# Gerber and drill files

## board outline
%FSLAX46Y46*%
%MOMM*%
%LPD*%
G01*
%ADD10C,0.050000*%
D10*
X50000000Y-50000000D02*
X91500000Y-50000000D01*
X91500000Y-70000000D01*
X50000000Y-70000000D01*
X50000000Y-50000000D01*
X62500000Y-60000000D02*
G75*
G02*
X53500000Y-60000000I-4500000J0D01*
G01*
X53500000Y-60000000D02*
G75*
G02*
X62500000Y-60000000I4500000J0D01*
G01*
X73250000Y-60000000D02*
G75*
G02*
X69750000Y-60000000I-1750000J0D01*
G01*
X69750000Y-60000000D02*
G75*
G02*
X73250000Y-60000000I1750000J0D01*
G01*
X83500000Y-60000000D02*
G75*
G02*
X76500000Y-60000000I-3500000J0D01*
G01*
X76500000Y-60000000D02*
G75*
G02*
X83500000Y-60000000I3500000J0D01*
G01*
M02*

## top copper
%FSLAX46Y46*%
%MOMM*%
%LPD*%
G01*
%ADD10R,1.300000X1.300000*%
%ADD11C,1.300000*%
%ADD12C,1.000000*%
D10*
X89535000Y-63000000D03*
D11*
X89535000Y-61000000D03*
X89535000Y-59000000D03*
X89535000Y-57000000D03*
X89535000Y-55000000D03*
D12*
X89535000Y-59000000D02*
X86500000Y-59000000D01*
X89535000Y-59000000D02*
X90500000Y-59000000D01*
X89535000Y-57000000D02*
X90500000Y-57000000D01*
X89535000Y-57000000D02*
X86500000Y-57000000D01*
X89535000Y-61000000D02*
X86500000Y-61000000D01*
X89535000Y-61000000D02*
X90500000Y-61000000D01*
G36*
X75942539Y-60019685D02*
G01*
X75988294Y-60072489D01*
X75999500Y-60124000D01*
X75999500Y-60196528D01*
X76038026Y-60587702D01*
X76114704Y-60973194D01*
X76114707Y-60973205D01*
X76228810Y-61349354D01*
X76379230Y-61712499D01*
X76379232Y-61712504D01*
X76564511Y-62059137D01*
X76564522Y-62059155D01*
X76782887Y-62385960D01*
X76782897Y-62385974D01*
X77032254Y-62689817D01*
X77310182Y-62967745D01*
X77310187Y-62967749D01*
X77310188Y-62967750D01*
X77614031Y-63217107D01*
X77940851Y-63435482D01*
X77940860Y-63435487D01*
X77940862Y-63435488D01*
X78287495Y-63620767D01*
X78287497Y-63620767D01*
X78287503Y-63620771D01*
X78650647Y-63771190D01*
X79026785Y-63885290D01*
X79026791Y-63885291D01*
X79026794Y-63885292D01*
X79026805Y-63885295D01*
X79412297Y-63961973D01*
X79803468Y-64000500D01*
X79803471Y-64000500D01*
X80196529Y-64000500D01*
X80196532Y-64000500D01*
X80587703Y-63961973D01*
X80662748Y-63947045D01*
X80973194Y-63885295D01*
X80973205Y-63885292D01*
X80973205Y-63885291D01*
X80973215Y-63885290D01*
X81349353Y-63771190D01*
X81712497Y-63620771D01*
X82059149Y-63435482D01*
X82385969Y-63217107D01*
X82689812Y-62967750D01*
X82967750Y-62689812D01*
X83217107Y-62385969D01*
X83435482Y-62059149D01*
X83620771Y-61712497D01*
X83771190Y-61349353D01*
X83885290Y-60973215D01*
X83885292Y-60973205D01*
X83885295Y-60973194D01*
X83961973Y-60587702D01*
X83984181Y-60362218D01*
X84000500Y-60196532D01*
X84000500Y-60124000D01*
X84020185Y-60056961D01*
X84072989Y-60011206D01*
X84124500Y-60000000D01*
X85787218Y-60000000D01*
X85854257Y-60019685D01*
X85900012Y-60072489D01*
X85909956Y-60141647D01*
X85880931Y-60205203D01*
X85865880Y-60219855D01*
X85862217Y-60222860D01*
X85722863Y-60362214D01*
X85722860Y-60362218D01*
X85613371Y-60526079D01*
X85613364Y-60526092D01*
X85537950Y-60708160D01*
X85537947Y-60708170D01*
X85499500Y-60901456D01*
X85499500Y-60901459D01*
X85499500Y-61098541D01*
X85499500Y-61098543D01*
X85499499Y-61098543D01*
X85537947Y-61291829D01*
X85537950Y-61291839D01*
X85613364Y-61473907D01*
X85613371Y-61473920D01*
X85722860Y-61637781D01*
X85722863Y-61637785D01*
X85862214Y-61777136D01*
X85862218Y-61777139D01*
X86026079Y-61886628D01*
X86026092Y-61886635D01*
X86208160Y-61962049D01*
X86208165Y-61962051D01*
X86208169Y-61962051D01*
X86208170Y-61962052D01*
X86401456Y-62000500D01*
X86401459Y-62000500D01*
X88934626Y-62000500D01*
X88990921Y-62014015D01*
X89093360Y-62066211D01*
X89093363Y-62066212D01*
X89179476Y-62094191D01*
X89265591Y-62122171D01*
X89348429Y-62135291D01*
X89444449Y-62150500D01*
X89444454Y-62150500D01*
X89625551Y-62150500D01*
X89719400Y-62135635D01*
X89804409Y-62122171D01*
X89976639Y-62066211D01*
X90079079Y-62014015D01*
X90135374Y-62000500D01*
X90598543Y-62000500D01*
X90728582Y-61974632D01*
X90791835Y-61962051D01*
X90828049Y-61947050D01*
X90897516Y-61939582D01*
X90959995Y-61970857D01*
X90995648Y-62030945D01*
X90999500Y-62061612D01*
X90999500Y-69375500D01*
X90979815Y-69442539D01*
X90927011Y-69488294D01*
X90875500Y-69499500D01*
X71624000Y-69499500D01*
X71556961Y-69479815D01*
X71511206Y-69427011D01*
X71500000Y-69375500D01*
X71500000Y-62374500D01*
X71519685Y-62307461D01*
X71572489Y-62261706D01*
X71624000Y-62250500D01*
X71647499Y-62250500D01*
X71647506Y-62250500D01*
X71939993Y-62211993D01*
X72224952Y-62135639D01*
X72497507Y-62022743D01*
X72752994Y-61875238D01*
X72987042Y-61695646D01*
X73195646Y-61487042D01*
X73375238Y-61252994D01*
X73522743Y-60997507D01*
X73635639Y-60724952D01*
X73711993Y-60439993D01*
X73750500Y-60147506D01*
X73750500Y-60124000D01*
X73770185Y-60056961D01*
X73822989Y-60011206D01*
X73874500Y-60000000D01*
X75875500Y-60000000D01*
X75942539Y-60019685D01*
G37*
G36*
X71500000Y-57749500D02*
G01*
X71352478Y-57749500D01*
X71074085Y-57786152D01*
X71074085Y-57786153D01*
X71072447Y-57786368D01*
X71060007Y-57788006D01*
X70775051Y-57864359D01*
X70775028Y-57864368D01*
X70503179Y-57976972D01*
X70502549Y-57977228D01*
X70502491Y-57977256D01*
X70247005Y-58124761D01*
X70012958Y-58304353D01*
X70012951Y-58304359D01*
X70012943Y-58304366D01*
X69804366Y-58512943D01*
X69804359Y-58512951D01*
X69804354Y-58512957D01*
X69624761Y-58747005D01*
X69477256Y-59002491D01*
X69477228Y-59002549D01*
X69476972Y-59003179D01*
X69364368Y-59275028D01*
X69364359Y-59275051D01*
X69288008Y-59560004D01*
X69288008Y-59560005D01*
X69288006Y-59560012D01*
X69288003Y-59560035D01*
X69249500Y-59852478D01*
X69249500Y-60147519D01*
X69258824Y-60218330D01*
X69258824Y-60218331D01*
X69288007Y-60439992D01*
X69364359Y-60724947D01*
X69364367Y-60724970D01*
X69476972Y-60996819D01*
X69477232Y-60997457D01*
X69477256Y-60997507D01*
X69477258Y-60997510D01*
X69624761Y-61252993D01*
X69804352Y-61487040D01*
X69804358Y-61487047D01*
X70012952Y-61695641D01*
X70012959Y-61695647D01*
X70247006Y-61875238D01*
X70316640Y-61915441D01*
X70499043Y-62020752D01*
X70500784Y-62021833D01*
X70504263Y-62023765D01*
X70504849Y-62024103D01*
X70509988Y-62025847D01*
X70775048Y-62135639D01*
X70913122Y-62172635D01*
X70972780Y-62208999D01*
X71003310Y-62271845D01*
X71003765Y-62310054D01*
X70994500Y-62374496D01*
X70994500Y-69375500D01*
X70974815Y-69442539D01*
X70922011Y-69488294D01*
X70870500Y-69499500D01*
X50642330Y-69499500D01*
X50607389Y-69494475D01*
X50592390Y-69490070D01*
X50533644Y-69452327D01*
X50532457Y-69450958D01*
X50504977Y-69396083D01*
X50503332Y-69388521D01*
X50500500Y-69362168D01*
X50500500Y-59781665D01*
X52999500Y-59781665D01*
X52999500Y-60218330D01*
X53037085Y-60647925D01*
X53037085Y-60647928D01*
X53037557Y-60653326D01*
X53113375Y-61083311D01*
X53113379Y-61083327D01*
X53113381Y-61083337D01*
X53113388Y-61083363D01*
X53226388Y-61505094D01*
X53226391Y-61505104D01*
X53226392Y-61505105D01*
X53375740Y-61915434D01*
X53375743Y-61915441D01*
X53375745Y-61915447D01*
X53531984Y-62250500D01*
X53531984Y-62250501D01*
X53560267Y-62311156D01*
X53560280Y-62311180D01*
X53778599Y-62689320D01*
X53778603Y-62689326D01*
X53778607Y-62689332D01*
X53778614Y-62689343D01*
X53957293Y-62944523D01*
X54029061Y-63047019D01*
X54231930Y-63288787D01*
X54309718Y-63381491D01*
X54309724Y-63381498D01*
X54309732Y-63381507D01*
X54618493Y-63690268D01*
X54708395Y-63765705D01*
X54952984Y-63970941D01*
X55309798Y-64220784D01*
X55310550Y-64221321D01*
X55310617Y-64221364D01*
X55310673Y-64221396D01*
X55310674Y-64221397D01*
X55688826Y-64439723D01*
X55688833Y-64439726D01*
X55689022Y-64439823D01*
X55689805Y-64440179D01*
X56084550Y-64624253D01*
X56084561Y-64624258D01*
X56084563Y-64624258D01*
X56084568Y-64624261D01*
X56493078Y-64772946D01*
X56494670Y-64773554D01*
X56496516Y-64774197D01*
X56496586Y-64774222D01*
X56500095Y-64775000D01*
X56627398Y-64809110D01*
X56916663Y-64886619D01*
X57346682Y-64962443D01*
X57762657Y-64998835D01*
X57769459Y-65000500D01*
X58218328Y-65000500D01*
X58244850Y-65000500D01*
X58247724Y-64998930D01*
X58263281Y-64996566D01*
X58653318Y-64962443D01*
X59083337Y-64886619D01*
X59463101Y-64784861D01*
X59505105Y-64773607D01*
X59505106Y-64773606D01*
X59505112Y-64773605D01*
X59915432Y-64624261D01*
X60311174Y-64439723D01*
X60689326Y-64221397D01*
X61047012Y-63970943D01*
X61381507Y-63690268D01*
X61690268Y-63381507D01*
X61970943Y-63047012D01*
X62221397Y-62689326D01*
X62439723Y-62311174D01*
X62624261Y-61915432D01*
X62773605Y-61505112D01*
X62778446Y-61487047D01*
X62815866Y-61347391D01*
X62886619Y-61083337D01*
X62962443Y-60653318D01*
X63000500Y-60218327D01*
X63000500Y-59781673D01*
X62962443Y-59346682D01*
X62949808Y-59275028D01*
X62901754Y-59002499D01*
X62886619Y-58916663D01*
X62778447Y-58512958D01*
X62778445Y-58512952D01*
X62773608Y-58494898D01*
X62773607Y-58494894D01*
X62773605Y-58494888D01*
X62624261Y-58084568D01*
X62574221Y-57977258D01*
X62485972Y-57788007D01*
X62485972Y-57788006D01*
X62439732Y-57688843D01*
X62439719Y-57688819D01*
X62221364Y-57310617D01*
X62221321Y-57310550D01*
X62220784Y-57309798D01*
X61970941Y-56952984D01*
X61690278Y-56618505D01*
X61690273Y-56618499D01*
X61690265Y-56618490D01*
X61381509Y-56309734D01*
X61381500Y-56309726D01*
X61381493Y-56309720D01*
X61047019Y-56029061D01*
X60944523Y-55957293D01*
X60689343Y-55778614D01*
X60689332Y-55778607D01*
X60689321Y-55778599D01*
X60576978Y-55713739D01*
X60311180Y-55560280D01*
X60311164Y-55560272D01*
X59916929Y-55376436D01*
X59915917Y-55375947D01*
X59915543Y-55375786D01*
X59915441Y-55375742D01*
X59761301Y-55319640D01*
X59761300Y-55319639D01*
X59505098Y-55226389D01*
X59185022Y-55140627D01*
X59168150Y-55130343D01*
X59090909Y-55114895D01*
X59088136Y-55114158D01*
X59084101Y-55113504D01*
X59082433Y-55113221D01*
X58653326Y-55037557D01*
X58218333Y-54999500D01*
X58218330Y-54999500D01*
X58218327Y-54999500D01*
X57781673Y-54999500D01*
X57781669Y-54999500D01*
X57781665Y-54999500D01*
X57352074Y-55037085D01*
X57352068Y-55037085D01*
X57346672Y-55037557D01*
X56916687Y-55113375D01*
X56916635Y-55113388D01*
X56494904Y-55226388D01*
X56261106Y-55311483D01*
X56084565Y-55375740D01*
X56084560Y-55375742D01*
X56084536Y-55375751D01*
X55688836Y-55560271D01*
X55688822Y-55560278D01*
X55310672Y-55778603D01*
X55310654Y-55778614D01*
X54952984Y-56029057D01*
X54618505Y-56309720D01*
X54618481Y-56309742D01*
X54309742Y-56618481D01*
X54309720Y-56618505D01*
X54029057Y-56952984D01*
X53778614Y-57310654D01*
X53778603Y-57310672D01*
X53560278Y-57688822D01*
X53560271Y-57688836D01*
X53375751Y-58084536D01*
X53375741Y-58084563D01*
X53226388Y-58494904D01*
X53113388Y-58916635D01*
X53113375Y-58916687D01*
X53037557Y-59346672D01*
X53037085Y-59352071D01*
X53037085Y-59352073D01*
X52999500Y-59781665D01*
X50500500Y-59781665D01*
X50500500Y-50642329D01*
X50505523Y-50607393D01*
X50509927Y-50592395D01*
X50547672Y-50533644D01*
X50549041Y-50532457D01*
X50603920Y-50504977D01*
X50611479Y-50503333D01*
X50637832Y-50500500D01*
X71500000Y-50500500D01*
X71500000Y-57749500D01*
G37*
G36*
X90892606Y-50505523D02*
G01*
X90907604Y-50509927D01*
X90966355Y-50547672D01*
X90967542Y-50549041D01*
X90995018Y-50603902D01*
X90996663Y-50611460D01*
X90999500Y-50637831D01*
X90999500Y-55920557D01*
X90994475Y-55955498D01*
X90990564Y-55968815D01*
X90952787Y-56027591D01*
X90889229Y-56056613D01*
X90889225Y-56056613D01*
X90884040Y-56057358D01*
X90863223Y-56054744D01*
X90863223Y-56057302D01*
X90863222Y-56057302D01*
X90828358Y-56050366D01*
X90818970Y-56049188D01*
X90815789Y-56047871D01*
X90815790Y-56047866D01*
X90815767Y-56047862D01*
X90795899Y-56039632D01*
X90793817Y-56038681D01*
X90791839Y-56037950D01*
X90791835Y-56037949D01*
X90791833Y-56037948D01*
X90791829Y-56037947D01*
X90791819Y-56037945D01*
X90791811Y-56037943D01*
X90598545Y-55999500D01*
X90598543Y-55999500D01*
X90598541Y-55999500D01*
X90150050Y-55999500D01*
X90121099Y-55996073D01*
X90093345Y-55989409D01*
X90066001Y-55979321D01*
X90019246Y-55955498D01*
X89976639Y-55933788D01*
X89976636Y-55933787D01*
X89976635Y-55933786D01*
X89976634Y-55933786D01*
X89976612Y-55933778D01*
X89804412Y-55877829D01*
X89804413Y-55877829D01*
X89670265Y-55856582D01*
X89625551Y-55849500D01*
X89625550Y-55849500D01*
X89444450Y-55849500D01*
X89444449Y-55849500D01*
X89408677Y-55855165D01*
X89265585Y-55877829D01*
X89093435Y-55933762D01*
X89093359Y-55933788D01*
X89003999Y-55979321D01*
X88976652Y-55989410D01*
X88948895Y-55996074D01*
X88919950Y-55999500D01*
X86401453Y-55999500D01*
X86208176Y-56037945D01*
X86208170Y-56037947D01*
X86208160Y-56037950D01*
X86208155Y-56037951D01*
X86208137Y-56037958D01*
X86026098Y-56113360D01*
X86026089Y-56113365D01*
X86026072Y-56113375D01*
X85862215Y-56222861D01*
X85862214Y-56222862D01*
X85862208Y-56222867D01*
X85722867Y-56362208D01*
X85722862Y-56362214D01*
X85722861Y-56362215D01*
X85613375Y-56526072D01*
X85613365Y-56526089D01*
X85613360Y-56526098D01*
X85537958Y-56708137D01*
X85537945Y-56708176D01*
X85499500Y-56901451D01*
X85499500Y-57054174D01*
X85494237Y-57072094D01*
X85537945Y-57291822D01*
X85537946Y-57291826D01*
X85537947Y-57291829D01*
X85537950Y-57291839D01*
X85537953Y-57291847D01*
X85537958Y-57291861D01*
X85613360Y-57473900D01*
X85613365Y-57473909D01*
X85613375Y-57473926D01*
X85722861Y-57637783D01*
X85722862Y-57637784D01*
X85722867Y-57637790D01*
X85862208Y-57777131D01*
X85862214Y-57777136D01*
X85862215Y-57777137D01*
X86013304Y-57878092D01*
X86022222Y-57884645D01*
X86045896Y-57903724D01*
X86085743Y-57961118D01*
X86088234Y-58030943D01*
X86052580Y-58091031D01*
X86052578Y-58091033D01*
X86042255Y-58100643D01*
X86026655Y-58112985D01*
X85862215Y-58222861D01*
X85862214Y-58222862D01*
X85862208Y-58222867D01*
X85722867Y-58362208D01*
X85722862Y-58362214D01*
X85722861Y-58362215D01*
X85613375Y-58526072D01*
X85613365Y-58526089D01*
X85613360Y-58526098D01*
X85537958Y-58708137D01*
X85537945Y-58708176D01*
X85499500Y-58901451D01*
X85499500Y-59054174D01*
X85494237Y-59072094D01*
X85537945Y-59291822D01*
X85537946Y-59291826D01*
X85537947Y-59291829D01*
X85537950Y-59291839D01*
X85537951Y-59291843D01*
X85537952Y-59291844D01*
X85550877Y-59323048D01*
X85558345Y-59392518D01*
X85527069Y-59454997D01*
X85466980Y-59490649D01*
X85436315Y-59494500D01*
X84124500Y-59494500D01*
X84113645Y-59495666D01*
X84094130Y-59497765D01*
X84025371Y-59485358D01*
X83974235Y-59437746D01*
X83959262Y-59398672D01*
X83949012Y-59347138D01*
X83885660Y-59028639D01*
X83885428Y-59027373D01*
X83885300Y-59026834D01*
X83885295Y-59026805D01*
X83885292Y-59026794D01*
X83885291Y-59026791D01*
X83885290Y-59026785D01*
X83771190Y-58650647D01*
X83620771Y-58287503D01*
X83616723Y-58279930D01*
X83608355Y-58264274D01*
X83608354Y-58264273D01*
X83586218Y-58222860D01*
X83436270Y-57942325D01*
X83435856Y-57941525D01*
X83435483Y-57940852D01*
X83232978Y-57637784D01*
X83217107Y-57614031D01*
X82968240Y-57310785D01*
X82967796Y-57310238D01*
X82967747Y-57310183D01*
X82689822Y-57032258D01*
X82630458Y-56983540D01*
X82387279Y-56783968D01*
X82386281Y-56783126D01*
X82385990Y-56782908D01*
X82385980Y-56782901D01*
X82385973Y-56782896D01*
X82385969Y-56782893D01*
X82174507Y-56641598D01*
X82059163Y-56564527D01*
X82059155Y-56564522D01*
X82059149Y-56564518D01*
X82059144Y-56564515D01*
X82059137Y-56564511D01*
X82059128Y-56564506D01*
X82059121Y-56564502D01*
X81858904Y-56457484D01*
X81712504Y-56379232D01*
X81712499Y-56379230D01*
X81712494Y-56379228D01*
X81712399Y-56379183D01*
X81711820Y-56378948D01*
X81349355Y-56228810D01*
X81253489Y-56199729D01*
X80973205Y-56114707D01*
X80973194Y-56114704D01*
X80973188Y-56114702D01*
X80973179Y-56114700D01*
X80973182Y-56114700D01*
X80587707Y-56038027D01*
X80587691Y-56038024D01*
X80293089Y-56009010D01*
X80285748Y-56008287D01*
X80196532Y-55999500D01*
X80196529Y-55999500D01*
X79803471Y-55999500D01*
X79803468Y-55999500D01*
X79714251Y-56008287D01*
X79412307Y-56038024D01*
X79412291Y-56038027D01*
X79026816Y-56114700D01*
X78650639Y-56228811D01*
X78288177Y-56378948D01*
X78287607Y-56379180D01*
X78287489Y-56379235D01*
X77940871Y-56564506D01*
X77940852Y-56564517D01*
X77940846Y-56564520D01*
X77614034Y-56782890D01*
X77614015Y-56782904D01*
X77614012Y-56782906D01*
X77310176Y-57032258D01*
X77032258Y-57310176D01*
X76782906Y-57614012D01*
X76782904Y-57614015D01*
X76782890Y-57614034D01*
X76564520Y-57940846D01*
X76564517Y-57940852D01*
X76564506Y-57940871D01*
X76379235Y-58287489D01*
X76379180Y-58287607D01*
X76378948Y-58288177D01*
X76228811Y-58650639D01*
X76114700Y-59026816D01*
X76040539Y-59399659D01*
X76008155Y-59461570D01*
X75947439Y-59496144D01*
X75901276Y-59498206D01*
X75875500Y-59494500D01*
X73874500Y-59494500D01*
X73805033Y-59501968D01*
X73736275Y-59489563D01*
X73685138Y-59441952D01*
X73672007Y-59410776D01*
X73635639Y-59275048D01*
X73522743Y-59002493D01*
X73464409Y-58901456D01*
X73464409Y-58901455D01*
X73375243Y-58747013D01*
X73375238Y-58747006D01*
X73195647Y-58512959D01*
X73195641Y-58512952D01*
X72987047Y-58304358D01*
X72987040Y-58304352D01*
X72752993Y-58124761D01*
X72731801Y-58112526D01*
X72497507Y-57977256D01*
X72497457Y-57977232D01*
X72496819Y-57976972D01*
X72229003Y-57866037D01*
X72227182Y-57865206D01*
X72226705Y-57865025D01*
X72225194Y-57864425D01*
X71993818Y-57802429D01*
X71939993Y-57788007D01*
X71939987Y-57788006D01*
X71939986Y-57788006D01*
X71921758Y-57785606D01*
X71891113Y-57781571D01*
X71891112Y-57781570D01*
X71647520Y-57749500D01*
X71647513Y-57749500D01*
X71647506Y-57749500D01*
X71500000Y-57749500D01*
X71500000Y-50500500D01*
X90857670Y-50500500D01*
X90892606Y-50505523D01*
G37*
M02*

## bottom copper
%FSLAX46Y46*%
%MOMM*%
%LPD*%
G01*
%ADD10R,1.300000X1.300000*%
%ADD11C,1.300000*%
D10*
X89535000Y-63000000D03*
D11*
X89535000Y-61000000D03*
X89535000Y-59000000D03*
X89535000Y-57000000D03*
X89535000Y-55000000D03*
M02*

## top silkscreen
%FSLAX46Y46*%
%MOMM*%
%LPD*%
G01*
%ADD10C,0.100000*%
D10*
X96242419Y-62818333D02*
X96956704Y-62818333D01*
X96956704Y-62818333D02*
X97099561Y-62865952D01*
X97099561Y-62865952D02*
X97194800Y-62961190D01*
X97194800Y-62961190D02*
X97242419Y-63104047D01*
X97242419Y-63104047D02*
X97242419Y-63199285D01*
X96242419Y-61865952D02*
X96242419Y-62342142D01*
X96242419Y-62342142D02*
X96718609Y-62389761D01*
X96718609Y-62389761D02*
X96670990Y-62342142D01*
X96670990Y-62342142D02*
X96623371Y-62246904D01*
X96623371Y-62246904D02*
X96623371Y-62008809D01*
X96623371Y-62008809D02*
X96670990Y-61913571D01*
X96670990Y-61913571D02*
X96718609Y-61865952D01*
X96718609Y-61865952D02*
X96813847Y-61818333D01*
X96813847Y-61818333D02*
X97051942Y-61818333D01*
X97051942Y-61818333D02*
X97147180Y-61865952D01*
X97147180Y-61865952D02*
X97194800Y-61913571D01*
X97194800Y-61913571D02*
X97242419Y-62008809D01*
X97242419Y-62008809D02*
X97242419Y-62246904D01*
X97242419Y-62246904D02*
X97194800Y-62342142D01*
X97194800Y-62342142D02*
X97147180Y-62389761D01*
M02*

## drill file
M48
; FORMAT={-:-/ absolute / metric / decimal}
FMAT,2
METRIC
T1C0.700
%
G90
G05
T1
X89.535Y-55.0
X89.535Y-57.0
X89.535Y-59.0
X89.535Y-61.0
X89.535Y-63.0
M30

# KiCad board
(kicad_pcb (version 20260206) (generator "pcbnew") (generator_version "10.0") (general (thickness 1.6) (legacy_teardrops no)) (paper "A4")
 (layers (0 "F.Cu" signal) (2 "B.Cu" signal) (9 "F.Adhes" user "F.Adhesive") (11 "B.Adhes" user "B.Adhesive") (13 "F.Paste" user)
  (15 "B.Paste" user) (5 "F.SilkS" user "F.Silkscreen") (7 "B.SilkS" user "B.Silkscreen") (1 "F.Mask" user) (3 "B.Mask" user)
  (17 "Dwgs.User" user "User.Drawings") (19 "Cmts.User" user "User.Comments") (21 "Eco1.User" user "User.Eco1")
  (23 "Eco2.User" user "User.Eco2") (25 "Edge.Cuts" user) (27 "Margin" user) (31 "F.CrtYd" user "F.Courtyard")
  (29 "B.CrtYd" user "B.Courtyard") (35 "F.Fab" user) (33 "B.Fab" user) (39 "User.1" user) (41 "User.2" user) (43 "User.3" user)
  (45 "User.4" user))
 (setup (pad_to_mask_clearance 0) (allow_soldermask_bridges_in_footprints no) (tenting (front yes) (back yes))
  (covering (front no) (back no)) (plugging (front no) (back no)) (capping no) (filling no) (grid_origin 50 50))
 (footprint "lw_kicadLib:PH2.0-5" (layer "F.Cu") (at 89.535 59 90)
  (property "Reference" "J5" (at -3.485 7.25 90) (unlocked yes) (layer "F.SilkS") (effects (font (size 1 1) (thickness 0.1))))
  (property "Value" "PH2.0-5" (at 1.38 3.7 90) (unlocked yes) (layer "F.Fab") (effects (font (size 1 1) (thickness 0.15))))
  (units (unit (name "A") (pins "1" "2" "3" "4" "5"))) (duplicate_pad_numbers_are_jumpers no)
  (pad "1" thru_hole rect (at -4 0 90) (size 1.3 1.3) (drill 0.7) (layers "*.Cu" "*.Mask") (remove_unused_layers no)
   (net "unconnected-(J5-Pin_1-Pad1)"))
  (pad "2" thru_hole circle (at -2 0 90) (size 1.3 1.3) (drill 0.7) (layers "*.Cu" "*.Mask") (remove_unused_layers no)
   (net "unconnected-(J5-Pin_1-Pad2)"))
  (pad "3" thru_hole circle (at 0 0 90) (size 1.3 1.3) (drill 0.7) (layers "*.Cu" "*.Mask") (remove_unused_layers no) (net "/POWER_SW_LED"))
  (pad "4" thru_hole circle (at 2 0 90) (size 1.3 1.3) (drill 0.7) (layers "*.Cu" "*.Mask") (remove_unused_layers no) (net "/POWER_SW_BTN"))
  (pad "5" thru_hole circle (at 4 0 90) (size 1.3 1.3) (drill 0.7) (layers "*.Cu" "*.Mask") (remove_unused_layers no) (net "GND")))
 (gr_rect (start 50 50) (end 91.5 70) (stroke (width 0.05) (type default)) (fill no) (layer "Edge.Cuts"))
 (gr_circle (center 58 60) (end 62.5 60) (stroke (width 0.05) (type default)) (fill no) (layer "Edge.Cuts"))
 (gr_circle (center 71.5 60) (end 73.25 60) (stroke (width 0.05) (type default)) (fill no) (layer "Edge.Cuts"))
 (gr_circle (center 80 60) (end 83.5 60) (stroke (width 0.05) (type default)) (fill no) (layer "Edge.Cuts"))
 (segment (start 89.535 59) (end 86.5 59) (width 1) (layer "F.Cu") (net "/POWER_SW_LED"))
 (segment (start 89.535 59) (end 90.5 59) (width 1) (layer "F.Cu") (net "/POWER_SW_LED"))
 (segment (start 89.535 57) (end 90.5 57) (width 1) (layer "F.Cu") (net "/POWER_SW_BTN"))
 (segment (start 89.535 57) (end 86.5 57) (width 1) (layer "F.Cu") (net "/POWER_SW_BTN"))
 (segment (start 89.535 61) (end 86.5 61) (width 1) (layer "F.Cu") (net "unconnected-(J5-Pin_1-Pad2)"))
 (segment (start 89.535 61) (end 90.5 61) (width 1) (layer "F.Cu") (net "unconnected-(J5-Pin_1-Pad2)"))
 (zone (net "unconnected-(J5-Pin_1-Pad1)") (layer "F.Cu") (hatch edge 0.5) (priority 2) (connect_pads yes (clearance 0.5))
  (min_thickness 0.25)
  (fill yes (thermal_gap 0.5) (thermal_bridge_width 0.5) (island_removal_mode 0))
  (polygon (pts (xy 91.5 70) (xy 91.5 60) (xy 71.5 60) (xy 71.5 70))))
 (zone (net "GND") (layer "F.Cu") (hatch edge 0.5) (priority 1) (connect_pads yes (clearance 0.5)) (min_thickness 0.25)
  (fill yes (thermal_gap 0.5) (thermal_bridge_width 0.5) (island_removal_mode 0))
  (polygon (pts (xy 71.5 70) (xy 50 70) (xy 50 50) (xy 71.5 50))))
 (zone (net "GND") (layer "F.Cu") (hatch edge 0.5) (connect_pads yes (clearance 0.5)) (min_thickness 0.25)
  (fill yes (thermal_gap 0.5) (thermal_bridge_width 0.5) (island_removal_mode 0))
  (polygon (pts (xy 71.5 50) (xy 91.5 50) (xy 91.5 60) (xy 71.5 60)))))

